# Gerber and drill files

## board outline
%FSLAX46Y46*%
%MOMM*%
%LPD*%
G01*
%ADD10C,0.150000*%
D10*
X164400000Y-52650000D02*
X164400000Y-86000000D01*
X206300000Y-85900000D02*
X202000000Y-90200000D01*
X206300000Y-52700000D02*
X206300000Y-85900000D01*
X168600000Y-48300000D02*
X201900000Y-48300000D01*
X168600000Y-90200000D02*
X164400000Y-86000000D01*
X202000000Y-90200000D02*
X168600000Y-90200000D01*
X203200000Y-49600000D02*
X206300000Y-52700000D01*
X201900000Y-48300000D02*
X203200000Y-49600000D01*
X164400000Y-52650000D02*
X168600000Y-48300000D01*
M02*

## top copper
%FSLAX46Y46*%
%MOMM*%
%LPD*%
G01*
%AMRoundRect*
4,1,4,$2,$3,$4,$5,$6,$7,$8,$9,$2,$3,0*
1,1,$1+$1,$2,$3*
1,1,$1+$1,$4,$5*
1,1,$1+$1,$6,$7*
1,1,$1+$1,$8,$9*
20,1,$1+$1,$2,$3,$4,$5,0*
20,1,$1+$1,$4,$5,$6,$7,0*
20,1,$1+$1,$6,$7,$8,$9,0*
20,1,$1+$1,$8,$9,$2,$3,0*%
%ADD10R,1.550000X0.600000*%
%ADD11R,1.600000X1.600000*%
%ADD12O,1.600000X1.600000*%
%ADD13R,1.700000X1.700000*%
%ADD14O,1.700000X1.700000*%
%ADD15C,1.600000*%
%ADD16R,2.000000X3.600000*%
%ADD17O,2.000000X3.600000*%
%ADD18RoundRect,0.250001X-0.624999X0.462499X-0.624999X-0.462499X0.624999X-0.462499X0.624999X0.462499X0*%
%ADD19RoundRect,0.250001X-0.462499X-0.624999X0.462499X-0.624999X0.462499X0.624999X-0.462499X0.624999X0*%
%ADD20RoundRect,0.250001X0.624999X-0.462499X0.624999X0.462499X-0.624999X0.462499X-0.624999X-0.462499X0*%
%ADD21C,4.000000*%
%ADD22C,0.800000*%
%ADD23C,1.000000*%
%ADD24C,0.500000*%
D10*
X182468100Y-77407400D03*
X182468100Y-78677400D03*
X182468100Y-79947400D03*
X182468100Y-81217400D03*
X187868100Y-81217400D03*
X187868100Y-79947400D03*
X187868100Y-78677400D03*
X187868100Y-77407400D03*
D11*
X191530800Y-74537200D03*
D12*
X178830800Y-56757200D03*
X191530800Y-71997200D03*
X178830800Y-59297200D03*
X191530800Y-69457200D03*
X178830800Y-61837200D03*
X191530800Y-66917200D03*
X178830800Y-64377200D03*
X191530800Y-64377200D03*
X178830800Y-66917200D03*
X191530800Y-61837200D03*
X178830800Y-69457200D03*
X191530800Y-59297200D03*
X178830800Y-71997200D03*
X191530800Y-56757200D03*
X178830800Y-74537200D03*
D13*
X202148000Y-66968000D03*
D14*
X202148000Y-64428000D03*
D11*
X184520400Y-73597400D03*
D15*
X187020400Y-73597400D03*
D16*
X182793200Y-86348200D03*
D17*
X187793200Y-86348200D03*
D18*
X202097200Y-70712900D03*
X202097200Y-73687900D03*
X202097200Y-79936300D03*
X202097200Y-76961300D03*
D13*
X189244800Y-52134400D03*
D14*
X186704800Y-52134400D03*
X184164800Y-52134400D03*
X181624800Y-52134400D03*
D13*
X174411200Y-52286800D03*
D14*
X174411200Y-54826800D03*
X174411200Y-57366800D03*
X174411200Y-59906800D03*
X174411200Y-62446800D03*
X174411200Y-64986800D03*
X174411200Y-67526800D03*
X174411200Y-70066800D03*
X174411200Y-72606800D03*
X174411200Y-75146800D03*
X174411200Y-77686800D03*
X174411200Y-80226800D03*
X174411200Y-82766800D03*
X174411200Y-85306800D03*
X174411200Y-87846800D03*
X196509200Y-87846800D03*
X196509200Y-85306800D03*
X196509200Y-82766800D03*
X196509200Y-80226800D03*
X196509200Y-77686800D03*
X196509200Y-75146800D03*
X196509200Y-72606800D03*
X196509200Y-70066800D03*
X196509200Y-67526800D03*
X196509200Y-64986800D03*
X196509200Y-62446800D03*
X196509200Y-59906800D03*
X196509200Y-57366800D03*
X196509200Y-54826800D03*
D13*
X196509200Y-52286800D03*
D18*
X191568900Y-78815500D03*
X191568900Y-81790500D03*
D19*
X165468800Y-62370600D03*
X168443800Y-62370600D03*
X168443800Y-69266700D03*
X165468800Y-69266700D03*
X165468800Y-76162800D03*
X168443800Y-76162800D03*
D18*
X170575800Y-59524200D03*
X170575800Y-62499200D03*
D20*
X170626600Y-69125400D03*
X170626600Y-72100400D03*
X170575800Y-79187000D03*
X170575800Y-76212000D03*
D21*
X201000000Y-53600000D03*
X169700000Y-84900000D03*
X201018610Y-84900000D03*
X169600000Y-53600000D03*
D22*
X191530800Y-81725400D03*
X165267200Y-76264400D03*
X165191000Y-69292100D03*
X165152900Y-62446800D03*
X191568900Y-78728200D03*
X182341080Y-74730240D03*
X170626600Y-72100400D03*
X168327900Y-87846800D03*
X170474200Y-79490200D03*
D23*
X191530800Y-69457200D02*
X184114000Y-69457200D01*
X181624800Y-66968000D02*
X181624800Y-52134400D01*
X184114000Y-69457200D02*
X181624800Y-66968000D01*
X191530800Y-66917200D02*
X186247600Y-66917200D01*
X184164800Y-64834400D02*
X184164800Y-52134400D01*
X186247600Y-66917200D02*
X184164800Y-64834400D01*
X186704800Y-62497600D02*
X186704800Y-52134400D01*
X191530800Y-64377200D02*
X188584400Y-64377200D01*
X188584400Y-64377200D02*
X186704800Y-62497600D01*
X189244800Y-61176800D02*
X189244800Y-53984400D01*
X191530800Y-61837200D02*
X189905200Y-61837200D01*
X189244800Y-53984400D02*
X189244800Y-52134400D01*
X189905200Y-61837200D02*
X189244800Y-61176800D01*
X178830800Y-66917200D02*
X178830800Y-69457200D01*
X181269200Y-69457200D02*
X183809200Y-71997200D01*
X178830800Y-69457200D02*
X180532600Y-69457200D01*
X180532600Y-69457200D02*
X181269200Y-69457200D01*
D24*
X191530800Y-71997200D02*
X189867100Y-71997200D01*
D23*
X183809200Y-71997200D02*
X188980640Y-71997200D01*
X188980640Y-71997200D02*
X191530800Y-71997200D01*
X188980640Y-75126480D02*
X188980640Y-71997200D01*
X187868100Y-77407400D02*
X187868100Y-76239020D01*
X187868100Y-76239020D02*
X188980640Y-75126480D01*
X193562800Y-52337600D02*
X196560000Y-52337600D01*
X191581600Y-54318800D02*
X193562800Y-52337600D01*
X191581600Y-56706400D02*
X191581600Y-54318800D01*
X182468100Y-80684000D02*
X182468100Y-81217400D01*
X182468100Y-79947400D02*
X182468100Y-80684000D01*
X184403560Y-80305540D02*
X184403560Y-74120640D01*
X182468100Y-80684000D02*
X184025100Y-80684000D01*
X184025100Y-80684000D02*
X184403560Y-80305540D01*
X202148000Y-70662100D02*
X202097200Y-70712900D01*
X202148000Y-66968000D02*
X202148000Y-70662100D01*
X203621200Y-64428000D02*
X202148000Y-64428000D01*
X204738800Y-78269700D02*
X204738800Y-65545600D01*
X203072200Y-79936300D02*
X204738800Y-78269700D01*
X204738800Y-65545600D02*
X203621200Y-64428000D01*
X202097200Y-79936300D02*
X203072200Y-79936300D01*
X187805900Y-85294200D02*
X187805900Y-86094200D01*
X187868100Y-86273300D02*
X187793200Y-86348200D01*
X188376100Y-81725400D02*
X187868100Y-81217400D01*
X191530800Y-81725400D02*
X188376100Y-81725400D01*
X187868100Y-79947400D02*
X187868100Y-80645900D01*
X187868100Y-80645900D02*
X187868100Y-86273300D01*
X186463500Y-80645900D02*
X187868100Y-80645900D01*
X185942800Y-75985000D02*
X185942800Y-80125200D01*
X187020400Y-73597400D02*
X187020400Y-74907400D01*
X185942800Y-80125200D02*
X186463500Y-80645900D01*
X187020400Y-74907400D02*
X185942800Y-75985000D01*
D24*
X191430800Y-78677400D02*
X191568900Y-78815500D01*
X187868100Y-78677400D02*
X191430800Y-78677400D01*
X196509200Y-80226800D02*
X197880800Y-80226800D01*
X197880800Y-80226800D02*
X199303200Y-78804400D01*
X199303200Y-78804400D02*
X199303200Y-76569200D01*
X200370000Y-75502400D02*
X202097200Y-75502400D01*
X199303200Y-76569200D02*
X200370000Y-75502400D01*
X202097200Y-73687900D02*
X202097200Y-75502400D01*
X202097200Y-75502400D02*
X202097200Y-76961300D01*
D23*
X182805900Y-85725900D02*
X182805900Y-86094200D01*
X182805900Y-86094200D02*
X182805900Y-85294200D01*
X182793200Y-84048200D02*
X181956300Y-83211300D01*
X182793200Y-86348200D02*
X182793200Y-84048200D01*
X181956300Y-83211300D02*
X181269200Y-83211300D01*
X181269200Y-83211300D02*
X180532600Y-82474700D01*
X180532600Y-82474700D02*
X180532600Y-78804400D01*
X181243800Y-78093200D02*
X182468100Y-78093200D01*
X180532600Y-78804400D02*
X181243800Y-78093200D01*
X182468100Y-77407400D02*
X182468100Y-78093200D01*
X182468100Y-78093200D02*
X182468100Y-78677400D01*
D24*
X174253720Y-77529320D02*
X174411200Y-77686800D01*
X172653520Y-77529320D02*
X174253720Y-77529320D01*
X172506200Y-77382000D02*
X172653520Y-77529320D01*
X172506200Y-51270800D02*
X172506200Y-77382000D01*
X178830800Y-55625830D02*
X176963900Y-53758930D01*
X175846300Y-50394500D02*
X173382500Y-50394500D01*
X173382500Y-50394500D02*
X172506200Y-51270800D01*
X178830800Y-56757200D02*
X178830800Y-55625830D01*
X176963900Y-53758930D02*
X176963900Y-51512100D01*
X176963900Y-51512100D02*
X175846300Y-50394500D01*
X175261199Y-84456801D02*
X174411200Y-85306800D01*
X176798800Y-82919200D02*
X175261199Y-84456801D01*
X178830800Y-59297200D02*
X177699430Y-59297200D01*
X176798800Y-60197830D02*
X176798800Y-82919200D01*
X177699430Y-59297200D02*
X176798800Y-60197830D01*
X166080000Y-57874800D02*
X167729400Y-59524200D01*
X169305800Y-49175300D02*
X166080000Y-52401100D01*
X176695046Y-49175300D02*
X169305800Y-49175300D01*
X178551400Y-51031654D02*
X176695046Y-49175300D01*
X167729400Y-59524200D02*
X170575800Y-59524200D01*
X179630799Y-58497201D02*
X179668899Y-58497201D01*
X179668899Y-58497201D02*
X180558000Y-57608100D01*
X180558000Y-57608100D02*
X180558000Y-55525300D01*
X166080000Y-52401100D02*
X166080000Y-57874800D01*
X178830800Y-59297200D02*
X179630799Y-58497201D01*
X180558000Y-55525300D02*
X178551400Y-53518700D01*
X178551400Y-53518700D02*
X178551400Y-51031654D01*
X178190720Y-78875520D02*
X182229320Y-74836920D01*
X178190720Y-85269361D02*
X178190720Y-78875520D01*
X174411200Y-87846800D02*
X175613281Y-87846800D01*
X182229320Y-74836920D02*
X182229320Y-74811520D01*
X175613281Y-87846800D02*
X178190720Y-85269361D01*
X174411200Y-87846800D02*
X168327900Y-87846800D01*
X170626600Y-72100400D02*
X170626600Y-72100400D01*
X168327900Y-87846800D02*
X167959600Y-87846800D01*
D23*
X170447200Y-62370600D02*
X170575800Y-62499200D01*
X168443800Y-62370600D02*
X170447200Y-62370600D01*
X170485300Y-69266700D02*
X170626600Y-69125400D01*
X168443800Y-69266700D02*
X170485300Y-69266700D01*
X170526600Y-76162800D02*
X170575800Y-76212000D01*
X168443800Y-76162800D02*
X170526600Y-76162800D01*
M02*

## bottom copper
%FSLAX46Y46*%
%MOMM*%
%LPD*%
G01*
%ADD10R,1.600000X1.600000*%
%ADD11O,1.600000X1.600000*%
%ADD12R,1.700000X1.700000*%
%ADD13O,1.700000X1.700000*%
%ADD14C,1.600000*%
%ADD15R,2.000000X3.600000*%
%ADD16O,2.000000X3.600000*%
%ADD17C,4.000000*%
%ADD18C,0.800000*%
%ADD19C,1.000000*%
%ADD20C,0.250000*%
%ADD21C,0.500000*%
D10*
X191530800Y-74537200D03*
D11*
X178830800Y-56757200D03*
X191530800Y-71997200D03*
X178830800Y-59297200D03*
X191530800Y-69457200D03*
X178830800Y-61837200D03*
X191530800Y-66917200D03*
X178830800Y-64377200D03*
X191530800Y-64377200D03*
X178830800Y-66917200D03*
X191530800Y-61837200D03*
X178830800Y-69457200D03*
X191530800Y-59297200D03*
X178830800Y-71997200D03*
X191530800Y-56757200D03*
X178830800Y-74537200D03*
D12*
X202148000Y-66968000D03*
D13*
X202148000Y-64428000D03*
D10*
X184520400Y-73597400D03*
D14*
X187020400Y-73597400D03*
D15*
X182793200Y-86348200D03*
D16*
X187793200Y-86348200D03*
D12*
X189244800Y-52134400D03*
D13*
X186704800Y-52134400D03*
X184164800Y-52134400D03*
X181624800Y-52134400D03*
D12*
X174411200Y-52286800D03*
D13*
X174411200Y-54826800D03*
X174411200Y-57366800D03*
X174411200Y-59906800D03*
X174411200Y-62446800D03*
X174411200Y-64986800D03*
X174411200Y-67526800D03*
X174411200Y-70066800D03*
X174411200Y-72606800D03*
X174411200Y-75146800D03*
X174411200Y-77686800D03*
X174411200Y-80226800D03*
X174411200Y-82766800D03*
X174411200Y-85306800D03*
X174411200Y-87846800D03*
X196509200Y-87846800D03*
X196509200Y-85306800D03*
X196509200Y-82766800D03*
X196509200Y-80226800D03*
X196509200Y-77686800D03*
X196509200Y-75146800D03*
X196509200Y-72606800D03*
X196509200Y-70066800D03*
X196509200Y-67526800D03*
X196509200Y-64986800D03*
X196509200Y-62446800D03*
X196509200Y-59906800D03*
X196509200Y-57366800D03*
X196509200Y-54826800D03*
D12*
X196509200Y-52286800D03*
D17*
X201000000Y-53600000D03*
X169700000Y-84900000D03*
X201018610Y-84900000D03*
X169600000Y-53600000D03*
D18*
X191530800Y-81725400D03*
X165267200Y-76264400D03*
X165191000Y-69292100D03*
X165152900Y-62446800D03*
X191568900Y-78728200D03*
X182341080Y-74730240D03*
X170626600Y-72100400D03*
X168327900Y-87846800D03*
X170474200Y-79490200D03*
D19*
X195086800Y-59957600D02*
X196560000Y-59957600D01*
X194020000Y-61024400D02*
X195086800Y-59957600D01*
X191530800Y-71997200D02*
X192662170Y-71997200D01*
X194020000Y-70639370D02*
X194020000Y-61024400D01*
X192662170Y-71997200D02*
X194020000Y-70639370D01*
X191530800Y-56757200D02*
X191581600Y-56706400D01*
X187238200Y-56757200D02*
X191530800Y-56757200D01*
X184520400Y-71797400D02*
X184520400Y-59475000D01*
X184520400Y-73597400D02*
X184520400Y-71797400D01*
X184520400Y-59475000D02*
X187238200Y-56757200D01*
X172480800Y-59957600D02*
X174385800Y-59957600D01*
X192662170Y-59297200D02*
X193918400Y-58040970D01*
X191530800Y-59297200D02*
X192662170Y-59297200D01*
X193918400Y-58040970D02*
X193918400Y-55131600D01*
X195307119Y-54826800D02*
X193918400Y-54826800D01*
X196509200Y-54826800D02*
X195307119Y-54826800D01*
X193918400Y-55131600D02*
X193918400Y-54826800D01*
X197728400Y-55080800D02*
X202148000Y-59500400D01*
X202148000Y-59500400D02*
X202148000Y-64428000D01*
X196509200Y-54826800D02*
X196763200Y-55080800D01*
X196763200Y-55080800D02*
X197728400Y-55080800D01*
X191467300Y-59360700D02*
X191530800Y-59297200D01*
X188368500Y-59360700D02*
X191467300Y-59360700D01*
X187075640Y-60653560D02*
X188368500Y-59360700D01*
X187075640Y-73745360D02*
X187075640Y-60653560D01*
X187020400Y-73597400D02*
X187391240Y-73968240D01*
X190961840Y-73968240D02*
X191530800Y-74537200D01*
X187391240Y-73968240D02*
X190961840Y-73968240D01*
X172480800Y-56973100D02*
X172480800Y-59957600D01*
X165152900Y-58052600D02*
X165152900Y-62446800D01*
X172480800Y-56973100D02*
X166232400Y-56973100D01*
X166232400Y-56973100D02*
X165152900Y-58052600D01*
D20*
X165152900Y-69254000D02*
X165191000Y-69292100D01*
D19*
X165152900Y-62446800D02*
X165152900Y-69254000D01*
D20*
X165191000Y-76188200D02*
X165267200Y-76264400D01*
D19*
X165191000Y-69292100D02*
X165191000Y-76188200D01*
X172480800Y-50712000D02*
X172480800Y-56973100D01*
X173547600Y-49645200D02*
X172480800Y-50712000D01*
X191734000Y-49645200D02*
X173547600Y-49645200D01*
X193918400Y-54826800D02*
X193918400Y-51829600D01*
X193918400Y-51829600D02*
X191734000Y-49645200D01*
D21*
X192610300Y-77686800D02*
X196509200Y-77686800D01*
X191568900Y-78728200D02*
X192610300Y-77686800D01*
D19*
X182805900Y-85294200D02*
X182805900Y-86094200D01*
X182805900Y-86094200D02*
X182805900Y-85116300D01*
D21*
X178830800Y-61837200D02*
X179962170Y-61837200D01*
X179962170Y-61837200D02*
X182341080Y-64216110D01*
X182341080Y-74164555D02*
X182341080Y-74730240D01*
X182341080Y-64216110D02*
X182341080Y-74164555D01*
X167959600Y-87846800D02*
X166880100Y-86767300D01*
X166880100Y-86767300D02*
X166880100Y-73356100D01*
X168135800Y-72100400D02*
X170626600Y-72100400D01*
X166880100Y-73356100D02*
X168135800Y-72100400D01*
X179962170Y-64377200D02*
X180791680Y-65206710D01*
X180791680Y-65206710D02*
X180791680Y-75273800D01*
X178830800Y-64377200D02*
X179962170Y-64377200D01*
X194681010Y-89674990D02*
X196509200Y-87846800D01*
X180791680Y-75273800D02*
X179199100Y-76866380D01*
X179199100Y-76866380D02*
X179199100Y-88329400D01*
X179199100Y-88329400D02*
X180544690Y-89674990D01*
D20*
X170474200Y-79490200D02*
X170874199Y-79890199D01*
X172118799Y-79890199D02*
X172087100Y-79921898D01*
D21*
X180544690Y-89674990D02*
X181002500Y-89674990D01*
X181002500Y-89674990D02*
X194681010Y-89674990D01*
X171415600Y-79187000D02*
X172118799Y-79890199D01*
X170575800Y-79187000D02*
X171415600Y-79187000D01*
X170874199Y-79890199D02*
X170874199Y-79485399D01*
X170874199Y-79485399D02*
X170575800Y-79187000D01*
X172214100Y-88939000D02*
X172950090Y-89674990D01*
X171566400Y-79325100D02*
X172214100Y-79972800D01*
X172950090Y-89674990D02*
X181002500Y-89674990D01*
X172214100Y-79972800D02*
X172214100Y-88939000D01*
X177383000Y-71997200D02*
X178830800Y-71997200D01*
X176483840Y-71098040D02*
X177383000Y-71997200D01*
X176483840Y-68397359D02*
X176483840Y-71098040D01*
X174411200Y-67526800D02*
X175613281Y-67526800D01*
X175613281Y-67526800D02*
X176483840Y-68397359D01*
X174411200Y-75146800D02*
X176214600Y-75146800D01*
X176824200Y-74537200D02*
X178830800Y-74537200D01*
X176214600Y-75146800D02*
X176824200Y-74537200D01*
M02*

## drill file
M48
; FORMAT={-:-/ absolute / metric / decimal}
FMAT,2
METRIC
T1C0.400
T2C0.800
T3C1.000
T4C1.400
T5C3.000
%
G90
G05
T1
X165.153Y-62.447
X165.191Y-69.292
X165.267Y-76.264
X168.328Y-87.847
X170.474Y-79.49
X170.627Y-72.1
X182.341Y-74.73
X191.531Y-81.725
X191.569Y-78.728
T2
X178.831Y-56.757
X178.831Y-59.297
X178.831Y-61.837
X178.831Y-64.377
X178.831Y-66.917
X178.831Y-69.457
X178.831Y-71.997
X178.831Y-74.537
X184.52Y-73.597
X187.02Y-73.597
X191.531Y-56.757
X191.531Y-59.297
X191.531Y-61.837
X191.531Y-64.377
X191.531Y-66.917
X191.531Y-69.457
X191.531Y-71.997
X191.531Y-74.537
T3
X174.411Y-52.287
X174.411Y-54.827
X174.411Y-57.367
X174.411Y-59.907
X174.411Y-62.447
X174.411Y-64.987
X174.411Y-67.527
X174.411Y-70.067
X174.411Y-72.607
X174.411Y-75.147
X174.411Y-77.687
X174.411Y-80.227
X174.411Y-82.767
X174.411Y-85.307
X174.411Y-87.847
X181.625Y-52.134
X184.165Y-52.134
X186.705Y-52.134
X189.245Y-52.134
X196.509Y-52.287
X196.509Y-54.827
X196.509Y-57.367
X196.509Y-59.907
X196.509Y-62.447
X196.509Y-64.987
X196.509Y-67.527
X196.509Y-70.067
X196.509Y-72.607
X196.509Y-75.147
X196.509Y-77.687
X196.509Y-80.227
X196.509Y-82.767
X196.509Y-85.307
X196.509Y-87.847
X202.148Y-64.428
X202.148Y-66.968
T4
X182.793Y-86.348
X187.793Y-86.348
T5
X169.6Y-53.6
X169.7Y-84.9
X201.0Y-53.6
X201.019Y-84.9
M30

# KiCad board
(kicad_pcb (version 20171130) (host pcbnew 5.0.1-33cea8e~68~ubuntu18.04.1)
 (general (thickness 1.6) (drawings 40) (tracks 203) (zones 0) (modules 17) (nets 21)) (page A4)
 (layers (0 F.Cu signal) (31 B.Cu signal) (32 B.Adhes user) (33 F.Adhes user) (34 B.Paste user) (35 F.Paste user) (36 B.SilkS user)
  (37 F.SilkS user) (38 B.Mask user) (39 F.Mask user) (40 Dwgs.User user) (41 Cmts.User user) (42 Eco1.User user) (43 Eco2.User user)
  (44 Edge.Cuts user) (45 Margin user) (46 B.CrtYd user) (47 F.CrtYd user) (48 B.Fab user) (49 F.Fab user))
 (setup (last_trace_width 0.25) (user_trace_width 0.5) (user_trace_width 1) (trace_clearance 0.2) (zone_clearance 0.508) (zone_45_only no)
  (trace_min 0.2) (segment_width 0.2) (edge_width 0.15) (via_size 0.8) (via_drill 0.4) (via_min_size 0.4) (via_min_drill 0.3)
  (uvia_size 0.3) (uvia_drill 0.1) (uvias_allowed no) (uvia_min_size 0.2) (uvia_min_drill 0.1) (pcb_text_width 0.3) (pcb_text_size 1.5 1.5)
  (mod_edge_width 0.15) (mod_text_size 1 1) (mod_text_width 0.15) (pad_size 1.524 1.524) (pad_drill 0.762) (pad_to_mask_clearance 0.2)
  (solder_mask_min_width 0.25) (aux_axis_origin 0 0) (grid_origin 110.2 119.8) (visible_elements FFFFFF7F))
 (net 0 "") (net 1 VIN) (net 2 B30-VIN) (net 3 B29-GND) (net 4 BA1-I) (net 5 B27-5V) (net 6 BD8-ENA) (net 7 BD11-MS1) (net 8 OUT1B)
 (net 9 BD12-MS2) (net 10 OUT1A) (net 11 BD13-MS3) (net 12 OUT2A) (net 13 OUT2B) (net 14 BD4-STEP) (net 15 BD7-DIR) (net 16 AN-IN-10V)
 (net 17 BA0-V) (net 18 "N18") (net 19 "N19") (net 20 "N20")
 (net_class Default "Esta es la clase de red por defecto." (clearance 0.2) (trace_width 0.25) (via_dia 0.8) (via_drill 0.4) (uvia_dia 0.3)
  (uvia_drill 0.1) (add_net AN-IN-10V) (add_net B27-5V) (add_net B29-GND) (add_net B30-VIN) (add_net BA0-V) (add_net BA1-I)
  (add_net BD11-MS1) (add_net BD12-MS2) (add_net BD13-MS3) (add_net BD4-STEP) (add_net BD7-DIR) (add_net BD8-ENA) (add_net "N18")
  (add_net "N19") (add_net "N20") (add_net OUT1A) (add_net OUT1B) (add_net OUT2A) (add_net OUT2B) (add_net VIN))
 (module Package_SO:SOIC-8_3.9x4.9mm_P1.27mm (layer F.Cu) (at 185.1681 79.3124)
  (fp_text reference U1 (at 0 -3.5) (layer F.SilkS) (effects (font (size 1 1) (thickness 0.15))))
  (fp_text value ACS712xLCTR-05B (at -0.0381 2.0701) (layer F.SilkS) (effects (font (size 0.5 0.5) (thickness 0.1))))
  (pad 1 smd rect (at -2.7 -1.905) (size 1.55 0.6) (layers F.Cu F.Paste F.Mask) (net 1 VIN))
  (pad 2 smd rect (at -2.7 -0.635) (size 1.55 0.6) (layers F.Cu F.Paste F.Mask) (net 1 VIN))
  (pad 3 smd rect (at -2.7 0.635) (size 1.55 0.6) (layers F.Cu F.Paste F.Mask) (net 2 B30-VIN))
  (pad 4 smd rect (at -2.7 1.905) (size 1.55 0.6) (layers F.Cu F.Paste F.Mask) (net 2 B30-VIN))
  (pad 5 smd rect (at 2.7 1.905) (size 1.55 0.6) (layers F.Cu F.Paste F.Mask) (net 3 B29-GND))
  (pad 6 smd rect (at 2.7 0.635) (size 1.55 0.6) (layers F.Cu F.Paste F.Mask) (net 3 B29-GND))
  (pad 7 smd rect (at 2.7 -0.635) (size 1.55 0.6) (layers F.Cu F.Paste F.Mask) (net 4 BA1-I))
  (pad 8 smd rect (at 2.7 -1.905) (size 1.55 0.6) (layers F.Cu F.Paste F.Mask) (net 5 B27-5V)))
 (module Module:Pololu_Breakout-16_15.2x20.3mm (layer F.Cu) (at 191.5308 74.5372 180)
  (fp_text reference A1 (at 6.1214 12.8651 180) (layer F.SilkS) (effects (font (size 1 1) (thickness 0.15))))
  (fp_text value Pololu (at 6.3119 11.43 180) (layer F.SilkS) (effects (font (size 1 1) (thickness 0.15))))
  (pad 1 thru_hole rect (at 0 0 180) (size 1.6 1.6) (drill 0.8) (layers *.Cu *.Mask) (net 3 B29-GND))
  (pad 9 thru_hole oval (at 12.7 17.78 180) (size 1.6 1.6) (drill 0.8) (layers *.Cu *.Mask) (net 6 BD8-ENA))
  (pad 2 thru_hole oval (at 0 2.54 180) (size 1.6 1.6) (drill 0.8) (layers *.Cu *.Mask) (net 5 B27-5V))
  (pad 10 thru_hole oval (at 12.7 15.24 180) (size 1.6 1.6) (drill 0.8) (layers *.Cu *.Mask) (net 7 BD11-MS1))
  (pad 3 thru_hole oval (at 0 5.08 180) (size 1.6 1.6) (drill 0.8) (layers *.Cu *.Mask) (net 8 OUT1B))
  (pad 11 thru_hole oval (at 12.7 12.7 180) (size 1.6 1.6) (drill 0.8) (layers *.Cu *.Mask) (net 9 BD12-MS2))
  (pad 4 thru_hole oval (at 0 7.62 180) (size 1.6 1.6) (drill 0.8) (layers *.Cu *.Mask) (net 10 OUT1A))
  (pad 12 thru_hole oval (at 12.7 10.16 180) (size 1.6 1.6) (drill 0.8) (layers *.Cu *.Mask) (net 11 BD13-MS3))
  (pad 5 thru_hole oval (at 0 10.16 180) (size 1.6 1.6) (drill 0.8) (layers *.Cu *.Mask) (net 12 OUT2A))
  (pad 13 thru_hole oval (at 12.7 7.62 180) (size 1.6 1.6) (drill 0.8) (layers *.Cu *.Mask) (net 5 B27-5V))
  (pad 6 thru_hole oval (at 0 12.7 180) (size 1.6 1.6) (drill 0.8) (layers *.Cu *.Mask) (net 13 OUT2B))
  (pad 14 thru_hole oval (at 12.7 5.08 180) (size 1.6 1.6) (drill 0.8) (layers *.Cu *.Mask) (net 5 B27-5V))
  (pad 7 thru_hole oval (at 0 15.24 180) (size 1.6 1.6) (drill 0.8) (layers *.Cu *.Mask) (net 3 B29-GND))
  (pad 15 thru_hole oval (at 12.7 2.54 180) (size 1.6 1.6) (drill 0.8) (layers *.Cu *.Mask) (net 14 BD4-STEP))
  (pad 8 thru_hole oval (at 0 17.78 180) (size 1.6 1.6) (drill 0.8) (layers *.Cu *.Mask) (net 2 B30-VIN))
  (pad 16 thru_hole oval (at 12.7 0 180) (size 1.6 1.6) (drill 0.8) (layers *.Cu *.Mask) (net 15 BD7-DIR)))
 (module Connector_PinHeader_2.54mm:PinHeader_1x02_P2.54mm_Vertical (layer F.Cu) (at 202.148 66.968 180)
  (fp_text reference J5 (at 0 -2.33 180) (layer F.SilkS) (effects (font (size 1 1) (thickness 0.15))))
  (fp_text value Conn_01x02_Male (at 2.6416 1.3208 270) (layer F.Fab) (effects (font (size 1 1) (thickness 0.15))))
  (pad 1 thru_hole rect (at 0 0 180) (size 1.7 1.7) (drill 1) (layers *.Cu *.Mask) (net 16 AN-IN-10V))
  (pad 2 thru_hole oval (at 0 2.54 180) (size 1.7 1.7) (drill 1) (layers *.Cu *.Mask) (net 3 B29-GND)))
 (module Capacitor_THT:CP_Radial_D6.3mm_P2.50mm (layer F.Cu) (at 184.5204 73.5974)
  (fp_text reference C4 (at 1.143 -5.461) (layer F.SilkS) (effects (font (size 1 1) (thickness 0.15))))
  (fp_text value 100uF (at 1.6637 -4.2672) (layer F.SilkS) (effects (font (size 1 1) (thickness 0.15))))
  (pad 1 thru_hole rect (at 0 0) (size 1.6 1.6) (drill 0.8) (layers *.Cu *.Mask) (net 2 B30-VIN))
  (pad 2 thru_hole circle (at 2.5 0) (size 1.6 1.6) (drill 0.8) (layers *.Cu *.Mask) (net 3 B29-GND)))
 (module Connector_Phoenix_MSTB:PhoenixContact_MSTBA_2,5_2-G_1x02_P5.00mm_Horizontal (layer F.Cu) (at 182.7932 86.3482)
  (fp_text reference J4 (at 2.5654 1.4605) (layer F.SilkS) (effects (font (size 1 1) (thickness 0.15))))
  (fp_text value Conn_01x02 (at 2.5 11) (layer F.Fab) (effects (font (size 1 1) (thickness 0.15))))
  (pad 1 thru_hole rect (at 0 0) (size 2 3.6) (drill 1.4) (layers *.Cu *.Mask) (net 1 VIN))
  (pad 2 thru_hole oval (at 5 0) (size 2 3.6) (drill 1.4) (layers *.Cu *.Mask) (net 3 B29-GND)))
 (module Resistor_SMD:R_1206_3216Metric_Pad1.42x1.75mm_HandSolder (layer F.Cu) (at 202.0972 72.2004 270)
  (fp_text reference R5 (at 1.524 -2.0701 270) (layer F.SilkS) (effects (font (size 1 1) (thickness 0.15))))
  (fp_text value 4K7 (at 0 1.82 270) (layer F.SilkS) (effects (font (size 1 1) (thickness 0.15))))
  (pad 1 smd roundrect (at -1.4875 0 270) (size 1.425 1.75) (layers F.Cu F.Paste F.Mask) (roundrect_rratio 0.175439) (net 16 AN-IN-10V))
  (pad 2 smd roundrect (at 1.4875 0 270) (size 1.425 1.75) (layers F.Cu F.Paste F.Mask) (roundrect_rratio 0.175439) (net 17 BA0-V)))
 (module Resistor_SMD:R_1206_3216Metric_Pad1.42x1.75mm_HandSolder (layer F.Cu) (at 202.0972 78.4488 270)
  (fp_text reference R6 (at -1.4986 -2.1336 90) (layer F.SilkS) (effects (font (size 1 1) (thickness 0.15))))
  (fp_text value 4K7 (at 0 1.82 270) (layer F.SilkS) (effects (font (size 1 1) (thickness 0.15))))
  (pad 2 smd roundrect (at 1.4875 0 270) (size 1.425 1.75) (layers F.Cu F.Paste F.Mask) (roundrect_rratio 0.175439) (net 3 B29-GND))
  (pad 1 smd roundrect (at -1.4875 0 270) (size 1.425 1.75) (layers F.Cu F.Paste F.Mask) (roundrect_rratio 0.175439) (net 17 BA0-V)))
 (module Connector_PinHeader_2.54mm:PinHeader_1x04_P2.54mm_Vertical (layer F.Cu) (at 189.2448 52.1344 270)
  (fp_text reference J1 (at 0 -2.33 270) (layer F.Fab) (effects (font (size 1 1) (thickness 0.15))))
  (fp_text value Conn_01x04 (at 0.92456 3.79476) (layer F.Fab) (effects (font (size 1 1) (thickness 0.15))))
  (pad 1 thru_hole rect (at 0 0 270) (size 1.7 1.7) (drill 1) (layers *.Cu *.Mask) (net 13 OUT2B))
  (pad 2 thru_hole oval (at 0 2.54 270) (size 1.7 1.7) (drill 1) (layers *.Cu *.Mask) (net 12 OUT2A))
  (pad 3 thru_hole oval (at 0 5.08 270) (size 1.7 1.7) (drill 1) (layers *.Cu *.Mask) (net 10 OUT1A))
  (pad 4 thru_hole oval (at 0 7.62 270) (size 1.7 1.7) (drill 1) (layers *.Cu *.Mask) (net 8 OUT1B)))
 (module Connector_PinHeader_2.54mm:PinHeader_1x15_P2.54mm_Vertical (layer B.Cu) (at 174.4112 52.2868 180)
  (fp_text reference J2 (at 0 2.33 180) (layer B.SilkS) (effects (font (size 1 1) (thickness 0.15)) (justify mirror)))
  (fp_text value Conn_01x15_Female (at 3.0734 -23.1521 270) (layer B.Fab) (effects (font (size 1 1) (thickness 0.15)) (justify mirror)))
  (pad 1 thru_hole rect (at 0 0 180) (size 1.7 1.7) (drill 1) (layers *.Cu *.Mask))
  (pad 2 thru_hole oval (at 0 -2.54 180) (size 1.7 1.7) (drill 1) (layers *.Cu *.Mask))
  (pad 3 thru_hole oval (at 0 -5.08 180) (size 1.7 1.7) (drill 1) (layers *.Cu *.Mask))
  (pad 4 thru_hole oval (at 0 -7.62 180) (size 1.7 1.7) (drill 1) (layers *.Cu *.Mask) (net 3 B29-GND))
  (pad 5 thru_hole oval (at 0 -10.16 180) (size 1.7 1.7) (drill 1) (layers *.Cu *.Mask))
  (pad 6 thru_hole oval (at 0 -12.7 180) (size 1.7 1.7) (drill 1) (layers *.Cu *.Mask))
  (pad 7 thru_hole oval (at 0 -15.24 180) (size 1.7 1.7) (drill 1) (layers *.Cu *.Mask) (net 14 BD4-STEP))
  (pad 8 thru_hole oval (at 0 -17.78 180) (size 1.7 1.7) (drill 1) (layers *.Cu *.Mask))
  (pad 9 thru_hole oval (at 0 -20.32 180) (size 1.7 1.7) (drill 1) (layers *.Cu *.Mask))
  (pad 10 thru_hole oval (at 0 -22.86 180) (size 1.7 1.7) (drill 1) (layers *.Cu *.Mask) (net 15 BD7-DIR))
  (pad 11 thru_hole oval (at 0 -25.4 180) (size 1.7 1.7) (drill 1) (layers *.Cu *.Mask) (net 6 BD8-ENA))
  (pad 12 thru_hole oval (at 0 -27.94 180) (size 1.7 1.7) (drill 1) (layers *.Cu *.Mask))
  (pad 13 thru_hole oval (at 0 -30.48 180) (size 1.7 1.7) (drill 1) (layers *.Cu *.Mask))
  (pad 14 thru_hole oval (at 0 -33.02 180) (size 1.7 1.7) (drill 1) (layers *.Cu *.Mask) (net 7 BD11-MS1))
  (pad 15 thru_hole oval (at 0 -35.56 180) (size 1.7 1.7) (drill 1) (layers *.Cu *.Mask) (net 9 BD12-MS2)))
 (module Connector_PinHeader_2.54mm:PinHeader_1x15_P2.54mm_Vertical (layer B.Cu) (at 196.5092 52.2868 180)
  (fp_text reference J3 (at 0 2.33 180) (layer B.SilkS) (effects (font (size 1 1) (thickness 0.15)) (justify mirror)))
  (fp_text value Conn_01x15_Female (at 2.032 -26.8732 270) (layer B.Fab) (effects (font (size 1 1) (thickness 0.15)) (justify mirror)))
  (pad 15 thru_hole oval (at 0 -35.56 180) (size 1.7 1.7) (drill 1) (layers *.Cu *.Mask) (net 11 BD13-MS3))
  (pad 14 thru_hole oval (at 0 -33.02 180) (size 1.7 1.7) (drill 1) (layers *.Cu *.Mask))
  (pad 13 thru_hole oval (at 0 -30.48 180) (size 1.7 1.7) (drill 1) (layers *.Cu *.Mask))
  (pad 12 thru_hole oval (at 0 -27.94 180) (size 1.7 1.7) (drill 1) (layers *.Cu *.Mask) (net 17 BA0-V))
  (pad 11 thru_hole oval (at 0 -25.4 180) (size 1.7 1.7) (drill 1) (layers *.Cu *.Mask) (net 4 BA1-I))
  (pad 10 thru_hole oval (at 0 -22.86 180) (size 1.7 1.7) (drill 1) (layers *.Cu *.Mask))
  (pad 9 thru_hole oval (at 0 -20.32 180) (size 1.7 1.7) (drill 1) (layers *.Cu *.Mask))
  (pad 8 thru_hole oval (at 0 -17.78 180) (size 1.7 1.7) (drill 1) (layers *.Cu *.Mask))
  (pad 7 thru_hole oval (at 0 -15.24 180) (size 1.7 1.7) (drill 1) (layers *.Cu *.Mask))
  (pad 6 thru_hole oval (at 0 -12.7 180) (size 1.7 1.7) (drill 1) (layers *.Cu *.Mask))
  (pad 5 thru_hole oval (at 0 -10.16 180) (size 1.7 1.7) (drill 1) (layers *.Cu *.Mask))
  (pad 4 thru_hole oval (at 0 -7.62 180) (size 1.7 1.7) (drill 1) (layers *.Cu *.Mask) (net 5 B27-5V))
  (pad 3 thru_hole oval (at 0 -5.08 180) (size 1.7 1.7) (drill 1) (layers *.Cu *.Mask))
  (pad 2 thru_hole oval (at 0 -2.54 180) (size 1.7 1.7) (drill 1) (layers *.Cu *.Mask) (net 3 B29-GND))
  (pad 1 thru_hole rect (at 0 0 180) (size 1.7 1.7) (drill 1) (layers *.Cu *.Mask) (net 2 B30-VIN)))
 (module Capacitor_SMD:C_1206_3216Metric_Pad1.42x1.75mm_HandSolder (layer F.Cu) (at 191.5689 80.303 270)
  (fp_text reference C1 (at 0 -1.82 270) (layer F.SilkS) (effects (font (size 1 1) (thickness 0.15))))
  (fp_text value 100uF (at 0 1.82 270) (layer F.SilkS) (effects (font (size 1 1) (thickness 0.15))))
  (pad 1 smd roundrect (at -1.4875 0 270) (size 1.425 1.75) (layers F.Cu F.Paste F.Mask) (roundrect_rratio 0.175439) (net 4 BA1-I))
  (pad 2 smd roundrect (at 1.4875 0 270) (size 1.425 1.75) (layers F.Cu F.Paste F.Mask) (roundrect_rratio 0.175439) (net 3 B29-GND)))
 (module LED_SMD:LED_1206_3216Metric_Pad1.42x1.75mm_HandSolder (layer F.Cu) (at 166.9563 62.3706)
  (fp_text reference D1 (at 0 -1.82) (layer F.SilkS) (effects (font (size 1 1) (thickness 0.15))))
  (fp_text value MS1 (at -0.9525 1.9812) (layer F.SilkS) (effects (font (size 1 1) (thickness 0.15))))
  (pad 1 smd roundrect (at -1.4875 0) (size 1.425 1.75) (layers F.Cu F.Paste F.Mask) (roundrect_rratio 0.175439) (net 3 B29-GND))
  (pad 2 smd roundrect (at 1.4875 0) (size 1.425 1.75) (layers F.Cu F.Paste F.Mask) (roundrect_rratio 0.175439) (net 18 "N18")))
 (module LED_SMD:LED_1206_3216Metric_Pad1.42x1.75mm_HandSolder (layer F.Cu) (at 166.9563 69.2667)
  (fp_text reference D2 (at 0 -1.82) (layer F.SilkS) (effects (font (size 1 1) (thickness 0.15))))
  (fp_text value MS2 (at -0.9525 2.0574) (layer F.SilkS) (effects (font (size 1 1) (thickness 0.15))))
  (pad 2 smd roundrect (at 1.4875 0) (size 1.425 1.75) (layers F.Cu F.Paste F.Mask) (roundrect_rratio 0.175439) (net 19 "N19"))
  (pad 1 smd roundrect (at -1.4875 0) (size 1.425 1.75) (layers F.Cu F.Paste F.Mask) (roundrect_rratio 0.175439) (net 3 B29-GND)))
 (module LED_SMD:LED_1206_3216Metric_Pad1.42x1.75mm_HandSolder (layer F.Cu) (at 166.9563 76.1628)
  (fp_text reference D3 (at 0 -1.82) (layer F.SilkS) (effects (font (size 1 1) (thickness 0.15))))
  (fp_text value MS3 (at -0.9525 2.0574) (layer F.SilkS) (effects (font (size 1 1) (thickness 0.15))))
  (pad 1 smd roundrect (at -1.4875 0) (size 1.425 1.75) (layers F.Cu F.Paste F.Mask) (roundrect_rratio 0.175439) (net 3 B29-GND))
  (pad 2 smd roundrect (at 1.4875 0) (size 1.425 1.75) (layers F.Cu F.Paste F.Mask) (roundrect_rratio 0.175439) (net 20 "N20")))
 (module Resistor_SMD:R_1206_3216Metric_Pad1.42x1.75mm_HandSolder (layer F.Cu) (at 170.5758 61.0117 270)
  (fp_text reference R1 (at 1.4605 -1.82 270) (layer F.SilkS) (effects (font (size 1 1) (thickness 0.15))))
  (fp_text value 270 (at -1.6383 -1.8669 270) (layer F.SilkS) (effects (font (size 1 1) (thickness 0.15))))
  (pad 1 smd roundrect (at -1.4875 0 270) (size 1.425 1.75) (layers F.Cu F.Paste F.Mask) (roundrect_rratio 0.175439) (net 7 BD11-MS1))
  (pad 2 smd roundrect (at 1.4875 0 270) (size 1.425 1.75) (layers F.Cu F.Paste F.Mask) (roundrect_rratio 0.175439) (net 18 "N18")))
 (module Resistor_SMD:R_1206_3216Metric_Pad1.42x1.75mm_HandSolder (layer F.Cu) (at 170.6266 70.6129 90)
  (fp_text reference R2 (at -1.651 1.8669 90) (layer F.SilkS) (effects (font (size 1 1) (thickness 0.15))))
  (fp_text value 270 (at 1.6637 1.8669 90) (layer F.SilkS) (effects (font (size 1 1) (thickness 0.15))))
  (pad 2 smd roundrect (at 1.4875 0 90) (size 1.425 1.75) (layers F.Cu F.Paste F.Mask) (roundrect_rratio 0.175439) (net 19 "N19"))
  (pad 1 smd roundrect (at -1.4875 0 90) (size 1.425 1.75) (layers F.Cu F.Paste F.Mask) (roundrect_rratio 0.175439) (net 9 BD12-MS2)))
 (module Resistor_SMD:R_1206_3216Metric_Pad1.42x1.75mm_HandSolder (layer F.Cu) (at 170.5758 77.6995 90)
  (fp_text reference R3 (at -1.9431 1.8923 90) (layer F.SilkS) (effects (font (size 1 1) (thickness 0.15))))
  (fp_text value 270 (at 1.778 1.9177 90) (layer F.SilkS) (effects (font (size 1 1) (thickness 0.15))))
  (pad 1 smd roundrect (at -1.4875 0 90) (size 1.425 1.75) (layers F.Cu F.Paste F.Mask) (roundrect_rratio 0.175439) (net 11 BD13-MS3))
  (pad 2 smd roundrect (at 1.4875 0 90) (size 1.425 1.75) (layers F.Cu F.Paste F.Mask) (roundrect_rratio 0.175439) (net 20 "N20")))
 (gr_line (start 164.4 52.65) (end 164.4 86) (layer Edge.Cuts) (width 0.15))
 (gr_line (start 206.3 85.9) (end 202 90.2) (layer Edge.Cuts) (width 0.15))
 (gr_line (start 206.3 52.7) (end 206.3 85.9) (layer Edge.Cuts) (width 0.15))
 (gr_line (start 168.6 48.3) (end 201.9 48.3) (layer Edge.Cuts) (width 0.15))
 (gr_line (start 168.6 90.2) (end 164.4 86) (layer Edge.Cuts) (width 0.15))
 (gr_line (start 202 90.2) (end 168.6 90.2) (layer Edge.Cuts) (width 0.15))
 (gr_line (start 203.2 49.6) (end 206.3 52.7) (layer Edge.Cuts) (width 0.15))
 (gr_line (start 201.9 48.3) (end 203.2 49.6) (layer Edge.Cuts) (width 0.15))
 (gr_line (start 164.4 52.65) (end 168.6 48.3) (layer Edge.Cuts) (width 0.15))
 (via (at 201 53.6) (size 4) (drill 3) (layers F.Cu B.Cu) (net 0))
 (via (at 169.7 84.9) (size 4) (drill 3) (layers F.Cu B.Cu) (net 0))
 (via (at 201.01861 84.9) (size 4) (drill 3) (layers F.Cu B.Cu) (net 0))
 (via (at 169.6 53.6) (size 4) (drill 3) (layers F.Cu B.Cu) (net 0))
 (segment (start 191.5308 69.4572) (end 184.114 69.4572) (width 1) (layer F.Cu) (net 8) (status 10))
 (segment (start 181.6248 66.968) (end 181.6248 52.1344) (width 1) (layer F.Cu) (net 8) (status 20))
 (segment (start 184.114 69.4572) (end 181.6248 66.968) (width 1) (layer F.Cu) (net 8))
 (segment (start 191.5308 66.9172) (end 186.2476 66.9172) (width 1) (layer F.Cu) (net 10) (status 10))
 (segment (start 184.1648 64.8344) (end 184.1648 52.1344) (width 1) (layer F.Cu) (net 10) (status 20))
 (segment (start 186.2476 66.9172) (end 184.1648 64.8344) (width 1) (layer F.Cu) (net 10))
 (segment (start 186.7048 62.4976) (end 186.7048 52.1344) (width 1) (layer F.Cu) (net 12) (status 20))
 (segment (start 191.5308 64.3772) (end 188.5844 64.3772) (width 1) (layer F.Cu) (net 12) (status 10))
 (segment (start 188.5844 64.3772) (end 186.7048 62.4976) (width 1) (layer F.Cu) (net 12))
 (segment (start 189.2448 61.1768) (end 189.2448 53.9844) (width 1) (layer F.Cu) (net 13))
 (segment (start 191.5308 61.8372) (end 189.9052 61.8372) (width 1) (layer F.Cu) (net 13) (status 10))
 (segment (start 189.2448 53.9844) (end 189.2448 52.1344) (width 1) (layer F.Cu) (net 13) (status 20))
 (segment (start 189.9052 61.8372) (end 189.2448 61.1768) (width 1) (layer F.Cu) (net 13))
 (segment (start 178.8308 66.9172) (end 178.8308 69.4572) (width 1) (layer F.Cu) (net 5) (status 30))
 (segment (start 195.0868 59.9576) (end 196.56 59.9576) (width 1) (layer B.Cu) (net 5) (status 20))
 (segment (start 194.02 61.0244) (end 195.0868 59.9576) (width 1) (layer B.Cu) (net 5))
 (segment (start 191.5308 71.9972) (end 192.66217 71.9972) (width 1) (layer B.Cu) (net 5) (status 10))
 (segment (start 194.02 70.63937) (end 194.02 61.0244) (width 1) (layer B.Cu) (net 5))
 (segment (start 192.66217 71.9972) (end 194.02 70.63937) (width 1) (layer B.Cu) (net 5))
 (segment (start 181.2692 69.4572) (end 183.8092 71.9972) (width 1) (layer F.Cu) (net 5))
 (segment (start 178.8308 69.4572) (end 180.5326 69.4572) (width 1) (layer F.Cu) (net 5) (status 10))
 (segment (start 180.5326 69.4572) (end 181.2692 69.4572) (width 1) (layer F.Cu) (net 5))
 (segment (start 191.5308 71.9972) (end 189.8671 71.9972) (width 0.5) (layer F.Cu) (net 5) (status 10))
 (segment (start 183.8092 71.9972) (end 188.98064 71.9972) (width 1) (layer F.Cu) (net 5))
 (segment (start 188.98064 71.9972) (end 191.5308 71.9972) (width 1) (layer F.Cu) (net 5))
 (segment (start 188.98064 75.12648) (end 188.98064 71.9972) (width 1) (layer F.Cu) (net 5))
 (segment (start 187.8681 77.4074) (end 187.8681 76.23902) (width 1) (layer F.Cu) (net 5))
 (segment (start 187.8681 76.23902) (end 188.98064 75.12648) (width 1) (layer F.Cu) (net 5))
 (segment (start 193.5628 52.3376) (end 196.56 52.3376) (width 1) (layer F.Cu) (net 2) (status 20))
 (segment (start 191.5816 54.3188) (end 193.5628 52.3376) (width 1) (layer F.Cu) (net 2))
 (segment (start 191.5308 56.7572) (end 191.5816 56.7064) (width 1) (layer B.Cu) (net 2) (status 30))
 (segment (start 191.5816 56.7064) (end 191.5816 54.3188) (width 1) (layer F.Cu) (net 2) (status 10))
 (segment (start 187.2382 56.7572) (end 191.5308 56.7572) (width 1) (layer B.Cu) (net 2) (status 20))
 (segment (start 182.4681 80.684) (end 182.4681 81.2174) (width 1) (layer F.Cu) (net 2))
 (segment (start 182.4681 79.9474) (end 182.4681 80.684) (width 1) (layer F.Cu) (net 2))
 (segment (start 184.5204 71.7974) (end 184.5204 59.475) (width 1) (layer B.Cu) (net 2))
 (segment (start 184.5204 73.5974) (end 184.5204 71.7974) (width 1) (layer B.Cu) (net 2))
 (segment (start 184.5204 59.475) (end 187.2382 56.7572) (width 1) (layer B.Cu) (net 2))
 (segment (start 184.40356 80.30554) (end 184.40356 74.12064) (width 1) (layer F.Cu) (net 2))
 (segment (start 182.4681 80.684) (end 184.0251 80.684) (width 1) (layer F.Cu) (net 2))
 (segment (start 184.0251 80.684) (end 184.40356 80.30554) (width 1) (layer F.Cu) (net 2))
 (segment (start 202.148 70.6621) (end 202.0972 70.7129) (width 1) (layer F.Cu) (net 16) (status 30))
 (segment (start 202.148 66.968) (end 202.148 70.6621) (width 1) (layer F.Cu) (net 16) (status 30))
 (via (at 191.5308 81.7254) (size 0.8) (drill 0.4) (layers F.Cu B.Cu) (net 3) (status 30))
 (segment (start 172.4808 59.9576) (end 174.3858 59.9576) (width 1) (layer B.Cu) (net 3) (status 20))
 (segment (start 192.66217 59.2972) (end 193.9184 58.04097) (width 1) (layer B.Cu) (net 3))
 (segment (start 191.5308 59.2972) (end 192.66217 59.2972) (width 1) (layer B.Cu) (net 3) (status 10))
 (segment (start 203.6212 64.428) (end 202.148 64.428) (width 1) (layer F.Cu) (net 3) (status 20))
 (segment (start 204.7388 78.2697) (end 204.7388 65.5456) (width 1) (layer F.Cu) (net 3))
 (segment (start 203.0722 79.9363) (end 204.7388 78.2697) (width 1) (layer F.Cu) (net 3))
 (segment (start 204.7388 65.5456) (end 203.6212 64.428) (width 1) (layer F.Cu) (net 3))
 (segment (start 202.0972 79.9363) (end 203.0722 79.9363) (width 1) (layer F.Cu) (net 3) (status 10))
 (segment (start 193.9184 58.04097) (end 193.9184 55.1316) (width 1) (layer B.Cu) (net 3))
 (segment (start 195.307119 54.8268) (end 193.9184 54.8268) (width 1) (layer B.Cu) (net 3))
 (segment (start 196.5092 54.8268) (end 195.307119 54.8268) (width 1) (layer B.Cu) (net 3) (status 10))
 (segment (start 193.9184 55.1316) (end 193.9184 54.8268) (width 1) (layer B.Cu) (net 3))
 (segment (start 197.7284 55.0808) (end 202.148 59.5004) (width 1) (layer B.Cu) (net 3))
 (segment (start 202.148 59.5004) (end 202.148 64.428) (width 1) (layer B.Cu) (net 3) (status 20))
 (segment (start 196.5092 54.8268) (end 196.7632 55.0808) (width 1) (layer B.Cu) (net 3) (status 30))
 (segment (start 196.7632 55.0808) (end 197.7284 55.0808) (width 1) (layer B.Cu) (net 3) (status 10))
 (segment (start 187.8059 85.2942) (end 187.8059 86.0942) (width 1) (layer F.Cu) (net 3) (status 30))
 (segment (start 187.8681 86.2733) (end 187.7932 86.3482) (width 1) (layer F.Cu) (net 3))
 (segment (start 188.3761 81.7254) (end 187.8681 81.2174) (width 1) (layer F.Cu) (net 3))
 (segment (start 191.5308 81.7254) (end 188.3761 81.7254) (width 1) (layer F.Cu) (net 3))
 (segment (start 187.8681 79.9474) (end 187.8681 80.6459) (width 1) (layer F.Cu) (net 3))
 (segment (start 187.8681 80.6459) (end 187.8681 86.2733) (width 1) (layer F.Cu) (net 3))
 (segment (start 186.4635 80.6459) (end 187.8681 80.6459) (width 1) (layer F.Cu) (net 3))
 (segment (start 185.9428 75.985) (end 185.9428 80.1252) (width 1) (layer F.Cu) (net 3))
 (segment (start 187.0204 73.5974) (end 187.0204 74.9074) (width 1) (layer F.Cu) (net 3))
 (segment (start 185.9428 80.1252) (end 186.4635 80.6459) (width 1) (layer F.Cu) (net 3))
 (segment (start 187.0204 74.9074) (end 185.9428 75.985) (width 1) (layer F.Cu) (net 3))
 (segment (start 191.4673 59.3607) (end 191.5308 59.2972) (width 1) (layer B.Cu) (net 3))
 (segment (start 188.3685 59.3607) (end 191.4673 59.3607) (width 1) (layer B.Cu) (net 3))
 (segment (start 187.07564 60.65356) (end 188.3685 59.3607) (width 1) (layer B.Cu) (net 3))
 (segment (start 187.07564 73.74536) (end 187.07564 60.65356) (width 1) (layer B.Cu) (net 3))
 (segment (start 187.0204 73.5974) (end 187.39124 73.96824) (width 1) (layer B.Cu) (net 3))
 (segment (start 190.96184 73.96824) (end 191.5308 74.5372) (width 1) (layer B.Cu) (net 3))
 (segment (start 187.39124 73.96824) (end 190.96184 73.96824) (width 1) (layer B.Cu) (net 3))
 (via (at 165.2672 76.2644) (size 0.8) (drill 0.4) (layers F.Cu B.Cu) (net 3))
 (via (at 165.191 69.2921) (size 0.8) (drill 0.4) (layers F.Cu B.Cu) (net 3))
 (via (at 165.1529 62.4468) (size 0.8) (drill 0.4) (layers F.Cu B.Cu) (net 3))
 (segment (start 172.4808 56.9731) (end 172.4808 59.9576) (width 1) (layer B.Cu) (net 3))
 (segment (start 165.1529 58.0526) (end 165.1529 62.4468) (width 1) (layer B.Cu) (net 3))
 (segment (start 172.4808 56.9731) (end 166.2324 56.9731) (width 1) (layer B.Cu) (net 3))
 (segment (start 166.2324 56.9731) (end 165.1529 58.0526) (width 1) (layer B.Cu) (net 3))
 (segment (start 165.1529 69.254) (end 165.191 69.2921) (width 0.25) (layer B.Cu) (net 3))
 (segment (start 165.1529 62.4468) (end 165.1529 69.254) (width 1) (layer B.Cu) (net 3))
 (segment (start 165.191 76.1882) (end 165.2672 76.2644) (width 0.25) (layer B.Cu) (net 3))
 (segment (start 165.191 69.2921) (end 165.191 76.1882) (width 1) (layer B.Cu) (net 3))
 (segment (start 172.4808 50.712) (end 172.4808 56.9731) (width 1) (layer B.Cu) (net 3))
 (segment (start 173.5476 49.6452) (end 172.4808 50.712) (width 1) (layer B.Cu) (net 3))
 (segment (start 191.734 49.6452) (end 173.5476 49.6452) (width 1) (layer B.Cu) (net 3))
 (segment (start 193.9184 54.8268) (end 193.9184 51.8296) (width 1) (layer B.Cu) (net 3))
 (segment (start 193.9184 51.8296) (end 191.734 49.6452) (width 1) (layer B.Cu) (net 3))
 (via (at 191.5689 78.7282) (size 0.8) (drill 0.4) (layers F.Cu B.Cu) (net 4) (status 30))
 (segment (start 192.6103 77.6868) (end 196.5092 77.6868) (width 0.5) (layer B.Cu) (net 4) (status 20))
 (segment (start 191.5689 78.7282) (end 192.6103 77.6868) (width 0.5) (layer B.Cu) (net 4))
 (segment (start 191.4308 78.6774) (end 191.5689 78.8155) (width 0.5) (layer F.Cu) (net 4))
 (segment (start 187.8681 78.6774) (end 191.4308 78.6774) (width 0.5) (layer F.Cu) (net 4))
 (segment (start 196.5092 80.2268) (end 197.8808 80.2268) (width 0.5) (layer F.Cu) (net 17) (status 10))
 (segment (start 197.8808 80.2268) (end 199.3032 78.8044) (width 0.5) (layer F.Cu) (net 17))
 (segment (start 199.3032 78.8044) (end 199.3032 76.5692) (width 0.5) (layer F.Cu) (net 17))
 (segment (start 200.37 75.5024) (end 202.0972 75.5024) (width 0.5) (layer F.Cu) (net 17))
 (segment (start 199.3032 76.5692) (end 200.37 75.5024) (width 0.5) (layer F.Cu) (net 17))
 (segment (start 202.0972 73.6879) (end 202.0972 75.5024) (width 0.5) (layer F.Cu) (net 17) (status 10))
 (segment (start 202.0972 75.5024) (end 202.0972 76.9613) (width 0.5) (layer F.Cu) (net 17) (status 20))
 (segment (start 182.8059 85.2942) (end 182.8059 86.0942) (width 1) (layer B.Cu) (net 1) (status 30))
 (segment (start 182.8059 86.0942) (end 182.8059 85.1163) (width 1) (layer B.Cu) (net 1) (status 30))
 (segment (start 182.8059 85.7259) (end 182.8059 86.0942) (width 1) (layer F.Cu) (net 1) (status 30))
 (segment (start 182.8059 86.0942) (end 182.8059 85.2942) (width 1) (layer F.Cu) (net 1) (status 30))
 (segment (start 182.7932 84.0482) (end 181.9563 83.2113) (width 1) (layer F.Cu) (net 1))
 (segment (start 182.7932 86.3482) (end 182.7932 84.0482) (width 1) (layer F.Cu) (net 1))
 (segment (start 181.9563 83.2113) (end 181.2692 83.2113) (width 1) (layer F.Cu) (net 1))
 (segment (start 181.2692 83.2113) (end 180.5326 82.4747) (width 1) (layer F.Cu) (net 1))
 (segment (start 180.5326 82.4747) (end 180.5326 78.8044) (width 1) (layer F.Cu) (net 1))
 (segment (start 181.2438 78.0932) (end 182.4681 78.0932) (width 1) (layer F.Cu) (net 1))
 (segment (start 180.5326 78.8044) (end 181.2438 78.0932) (width 1) (layer F.Cu) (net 1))
 (segment (start 182.4681 77.4074) (end 182.4681 78.0932) (width 1) (layer F.Cu) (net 1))
 (segment (start 182.4681 78.0932) (end 182.4681 78.6774) (width 1) (layer F.Cu) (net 1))
 (segment (start 174.25372 77.52932) (end 174.4112 77.6868) (width 0.5) (layer F.Cu) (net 6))
 (segment (start 172.65352 77.52932) (end 174.25372 77.52932) (width 0.5) (layer F.Cu) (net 6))
 (segment (start 172.5062 77.382) (end 172.65352 77.52932) (width 0.5) (layer F.Cu) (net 6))
 (segment (start 172.5062 51.2708) (end 172.5062 77.382) (width 0.5) (layer F.Cu) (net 6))
 (segment (start 178.8308 55.62583) (end 176.9639 53.75893) (width 0.5) (layer F.Cu) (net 6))
 (segment (start 175.8463 50.3945) (end 173.3825 50.3945) (width 0.5) (layer F.Cu) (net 6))
 (segment (start 173.3825 50.3945) (end 172.5062 51.2708) (width 0.5) (layer F.Cu) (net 6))
 (segment (start 178.8308 56.7572) (end 178.8308 55.62583) (width 0.5) (layer F.Cu) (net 6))
 (segment (start 176.9639 53.75893) (end 176.9639 51.5121) (width 0.5) (layer F.Cu) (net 6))
 (segment (start 176.9639 51.5121) (end 175.8463 50.3945) (width 0.5) (layer F.Cu) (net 6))
 (segment (start 175.261199 84.456801) (end 174.4112 85.3068) (width 0.5) (layer F.Cu) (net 7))
 (segment (start 176.7988 82.9192) (end 175.261199 84.456801) (width 0.5) (layer F.Cu) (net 7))
 (segment (start 178.8308 59.2972) (end 177.69943 59.2972) (width 0.5) (layer F.Cu) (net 7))
 (segment (start 176.7988 60.19783) (end 176.7988 82.9192) (width 0.5) (layer F.Cu) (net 7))
 (segment (start 177.69943 59.2972) (end 176.7988 60.19783) (width 0.5) (layer F.Cu) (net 7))
 (segment (start 166.08 57.8748) (end 167.7294 59.5242) (width 0.5) (layer F.Cu) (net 7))
 (segment (start 169.3058 49.1753) (end 166.08 52.4011) (width 0.5) (layer F.Cu) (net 7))
 (segment (start 176.695046 49.1753) (end 169.3058 49.1753) (width 0.5) (layer F.Cu) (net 7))
 (segment (start 178.5514 51.031654) (end 176.695046 49.1753) (width 0.5) (layer F.Cu) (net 7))
 (segment (start 167.7294 59.5242) (end 170.5758 59.5242) (width 0.5) (layer F.Cu) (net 7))
 (segment (start 179.630799 58.497201) (end 179.668899 58.497201) (width 0.5) (layer F.Cu) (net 7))
 (segment (start 179.668899 58.497201) (end 180.558 57.6081) (width 0.5) (layer F.Cu) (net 7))
 (segment (start 180.558 57.6081) (end 180.558 55.5253) (width 0.5) (layer F.Cu) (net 7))
 (segment (start 166.08 52.4011) (end 166.08 57.8748) (width 0.5) (layer F.Cu) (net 7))
 (segment (start 178.8308 59.2972) (end 179.630799 58.497201) (width 0.5) (layer F.Cu) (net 7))
 (segment (start 180.558 55.5253) (end 178.5514 53.5187) (width 0.5) (layer F.Cu) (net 7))
 (segment (start 178.5514 53.5187) (end 178.5514 51.031654) (width 0.5) (layer F.Cu) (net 7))
 (segment (start 178.19072 78.87552) (end 182.22932 74.83692) (width 0.5) (layer F.Cu) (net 9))
 (segment (start 178.19072 85.269361) (end 178.19072 78.87552) (width 0.5) (layer F.Cu) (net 9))
 (segment (start 174.4112 87.8468) (end 175.613281 87.8468) (width 0.5) (layer F.Cu) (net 9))
 (segment (start 182.22932 74.83692) (end 182.22932 74.81152) (width 0.5) (layer F.Cu) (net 9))
 (segment (start 175.613281 87.8468) (end 178.19072 85.269361) (width 0.5) (layer F.Cu) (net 9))
 (via (at 182.34108 74.73024) (size 0.8) (drill 0.4) (layers F.Cu B.Cu) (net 9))
 (segment (start 178.8308 61.8372) (end 179.96217 61.8372) (width 0.5) (layer B.Cu) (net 9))
 (segment (start 179.96217 61.8372) (end 182.34108 64.21611) (width 0.5) (layer B.Cu) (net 9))
 (segment (start 182.34108 74.164555) (end 182.34108 74.73024) (width 0.5) (layer B.Cu) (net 9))
 (segment (start 182.34108 64.21611) (end 182.34108 74.164555) (width 0.5) (layer B.Cu) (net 9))
 (segment (start 174.4112 87.8468) (end 168.3279 87.8468) (width 0.5) (layer F.Cu) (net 9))
 (segment (start 167.9596 87.8468) (end 166.8801 86.7673) (width 0.5) (layer B.Cu) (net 9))
 (segment (start 166.8801 86.7673) (end 166.8801 73.3561) (width 0.5) (layer B.Cu) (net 9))
 (segment (start 168.1358 72.1004) (end 170.6266 72.1004) (width 0.5) (layer B.Cu) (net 9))
 (segment (start 166.8801 73.3561) (end 168.1358 72.1004) (width 0.5) (layer B.Cu) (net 9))
 (segment (start 170.6266 72.1004) (end 170.6266 72.1004) (width 0.5) (layer F.Cu) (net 9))
 (via (at 170.6266 72.1004) (size 0.8) (drill 0.4) (layers F.Cu B.Cu) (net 9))
 (segment (start 168.3279 87.8468) (end 167.9596 87.8468) (width 0.5) (layer F.Cu) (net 9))
 (via (at 168.3279 87.8468) (size 0.8) (drill 0.4) (layers F.Cu B.Cu) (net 9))
 (via (at 170.4742 79.4902) (size 0.8) (drill 0.4) (layers F.Cu B.Cu) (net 11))
 (segment (start 179.96217 64.3772) (end 180.79168 65.20671) (width 0.5) (layer B.Cu) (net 11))
 (segment (start 180.79168 65.20671) (end 180.79168 75.2738) (width 0.5) (layer B.Cu) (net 11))
 (segment (start 178.8308 64.3772) (end 179.96217 64.3772) (width 0.5) (layer B.Cu) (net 11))
 (segment (start 194.68101 89.67499) (end 196.5092 87.8468) (width 0.5) (layer B.Cu) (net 11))
 (segment (start 180.79168 75.2738) (end 179.1991 76.86638) (width 0.5) (layer B.Cu) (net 11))
 (segment (start 179.1991 76.86638) (end 179.1991 88.3294) (width 0.5) (layer B.Cu) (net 11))
 (segment (start 179.1991 88.3294) (end 180.54469 89.67499) (width 0.5) (layer B.Cu) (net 11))
 (segment (start 170.4742 79.4902) (end 170.874199 79.890199) (width 0.25) (layer B.Cu) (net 11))
 (segment (start 172.118799 79.890199) (end 172.0871 79.921898) (width 0.25) (layer B.Cu) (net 11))
 (segment (start 180.54469 89.67499) (end 181.0025 89.67499) (width 0.5) (layer B.Cu) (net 11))
 (segment (start 181.0025 89.67499) (end 194.68101 89.67499) (width 0.5) (layer B.Cu) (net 11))
 (segment (start 171.4156 79.187) (end 172.118799 79.890199) (width 0.5) (layer B.Cu) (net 11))
 (segment (start 170.5758 79.187) (end 171.4156 79.187) (width 0.5) (layer B.Cu) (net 11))
 (segment (start 170.874199 79.890199) (end 170.874199 79.485399) (width 0.5) (layer B.Cu) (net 11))
 (segment (start 170.874199 79.485399) (end 170.5758 79.187) (width 0.5) (layer B.Cu) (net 11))
 (segment (start 172.2141 88.939) (end 172.95009 89.67499) (width 0.5) (layer B.Cu) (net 11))
 (segment (start 171.5664 79.3251) (end 172.2141 79.9728) (width 0.5) (layer B.Cu) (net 11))
 (segment (start 172.95009 89.67499) (end 181.0025 89.67499) (width 0.5) (layer B.Cu) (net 11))
 (segment (start 172.2141 79.9728) (end 172.2141 88.939) (width 0.5) (layer B.Cu) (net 11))
 (segment (start 177.383 71.9972) (end 178.8308 71.9972) (width 0.5) (layer B.Cu) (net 14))
 (segment (start 176.48384 71.09804) (end 177.383 71.9972) (width 0.5) (layer B.Cu) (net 14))
 (segment (start 176.48384 68.397359) (end 176.48384 71.09804) (width 0.5) (layer B.Cu) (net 14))
 (segment (start 174.4112 67.5268) (end 175.613281 67.5268) (width 0.5) (layer B.Cu) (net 14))
 (segment (start 175.613281 67.5268) (end 176.48384 68.397359) (width 0.5) (layer B.Cu) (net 14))
 (segment (start 174.4112 75.1468) (end 176.2146 75.1468) (width 0.5) (layer B.Cu) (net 15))
 (segment (start 176.8242 74.5372) (end 178.8308 74.5372) (width 0.5) (layer B.Cu) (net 15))
 (segment (start 176.2146 75.1468) (end 176.8242 74.5372) (width 0.5) (layer B.Cu) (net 15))
 (segment (start 170.4472 62.3706) (end 170.5758 62.4992) (width 1) (layer F.Cu) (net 18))
 (segment (start 168.4438 62.3706) (end 170.4472 62.3706) (width 1) (layer F.Cu) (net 18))
 (segment (start 170.4853 69.2667) (end 170.6266 69.1254) (width 1) (layer F.Cu) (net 19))
 (segment (start 168.4438 69.2667) (end 170.4853 69.2667) (width 1) (layer F.Cu) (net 19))
 (segment (start 170.5266 76.1628) (end 170.5758 76.212) (width 1) (layer F.Cu) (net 20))
 (segment (start 168.4438 76.1628) (end 170.5266 76.1628) (width 1) (layer F.Cu) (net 20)))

